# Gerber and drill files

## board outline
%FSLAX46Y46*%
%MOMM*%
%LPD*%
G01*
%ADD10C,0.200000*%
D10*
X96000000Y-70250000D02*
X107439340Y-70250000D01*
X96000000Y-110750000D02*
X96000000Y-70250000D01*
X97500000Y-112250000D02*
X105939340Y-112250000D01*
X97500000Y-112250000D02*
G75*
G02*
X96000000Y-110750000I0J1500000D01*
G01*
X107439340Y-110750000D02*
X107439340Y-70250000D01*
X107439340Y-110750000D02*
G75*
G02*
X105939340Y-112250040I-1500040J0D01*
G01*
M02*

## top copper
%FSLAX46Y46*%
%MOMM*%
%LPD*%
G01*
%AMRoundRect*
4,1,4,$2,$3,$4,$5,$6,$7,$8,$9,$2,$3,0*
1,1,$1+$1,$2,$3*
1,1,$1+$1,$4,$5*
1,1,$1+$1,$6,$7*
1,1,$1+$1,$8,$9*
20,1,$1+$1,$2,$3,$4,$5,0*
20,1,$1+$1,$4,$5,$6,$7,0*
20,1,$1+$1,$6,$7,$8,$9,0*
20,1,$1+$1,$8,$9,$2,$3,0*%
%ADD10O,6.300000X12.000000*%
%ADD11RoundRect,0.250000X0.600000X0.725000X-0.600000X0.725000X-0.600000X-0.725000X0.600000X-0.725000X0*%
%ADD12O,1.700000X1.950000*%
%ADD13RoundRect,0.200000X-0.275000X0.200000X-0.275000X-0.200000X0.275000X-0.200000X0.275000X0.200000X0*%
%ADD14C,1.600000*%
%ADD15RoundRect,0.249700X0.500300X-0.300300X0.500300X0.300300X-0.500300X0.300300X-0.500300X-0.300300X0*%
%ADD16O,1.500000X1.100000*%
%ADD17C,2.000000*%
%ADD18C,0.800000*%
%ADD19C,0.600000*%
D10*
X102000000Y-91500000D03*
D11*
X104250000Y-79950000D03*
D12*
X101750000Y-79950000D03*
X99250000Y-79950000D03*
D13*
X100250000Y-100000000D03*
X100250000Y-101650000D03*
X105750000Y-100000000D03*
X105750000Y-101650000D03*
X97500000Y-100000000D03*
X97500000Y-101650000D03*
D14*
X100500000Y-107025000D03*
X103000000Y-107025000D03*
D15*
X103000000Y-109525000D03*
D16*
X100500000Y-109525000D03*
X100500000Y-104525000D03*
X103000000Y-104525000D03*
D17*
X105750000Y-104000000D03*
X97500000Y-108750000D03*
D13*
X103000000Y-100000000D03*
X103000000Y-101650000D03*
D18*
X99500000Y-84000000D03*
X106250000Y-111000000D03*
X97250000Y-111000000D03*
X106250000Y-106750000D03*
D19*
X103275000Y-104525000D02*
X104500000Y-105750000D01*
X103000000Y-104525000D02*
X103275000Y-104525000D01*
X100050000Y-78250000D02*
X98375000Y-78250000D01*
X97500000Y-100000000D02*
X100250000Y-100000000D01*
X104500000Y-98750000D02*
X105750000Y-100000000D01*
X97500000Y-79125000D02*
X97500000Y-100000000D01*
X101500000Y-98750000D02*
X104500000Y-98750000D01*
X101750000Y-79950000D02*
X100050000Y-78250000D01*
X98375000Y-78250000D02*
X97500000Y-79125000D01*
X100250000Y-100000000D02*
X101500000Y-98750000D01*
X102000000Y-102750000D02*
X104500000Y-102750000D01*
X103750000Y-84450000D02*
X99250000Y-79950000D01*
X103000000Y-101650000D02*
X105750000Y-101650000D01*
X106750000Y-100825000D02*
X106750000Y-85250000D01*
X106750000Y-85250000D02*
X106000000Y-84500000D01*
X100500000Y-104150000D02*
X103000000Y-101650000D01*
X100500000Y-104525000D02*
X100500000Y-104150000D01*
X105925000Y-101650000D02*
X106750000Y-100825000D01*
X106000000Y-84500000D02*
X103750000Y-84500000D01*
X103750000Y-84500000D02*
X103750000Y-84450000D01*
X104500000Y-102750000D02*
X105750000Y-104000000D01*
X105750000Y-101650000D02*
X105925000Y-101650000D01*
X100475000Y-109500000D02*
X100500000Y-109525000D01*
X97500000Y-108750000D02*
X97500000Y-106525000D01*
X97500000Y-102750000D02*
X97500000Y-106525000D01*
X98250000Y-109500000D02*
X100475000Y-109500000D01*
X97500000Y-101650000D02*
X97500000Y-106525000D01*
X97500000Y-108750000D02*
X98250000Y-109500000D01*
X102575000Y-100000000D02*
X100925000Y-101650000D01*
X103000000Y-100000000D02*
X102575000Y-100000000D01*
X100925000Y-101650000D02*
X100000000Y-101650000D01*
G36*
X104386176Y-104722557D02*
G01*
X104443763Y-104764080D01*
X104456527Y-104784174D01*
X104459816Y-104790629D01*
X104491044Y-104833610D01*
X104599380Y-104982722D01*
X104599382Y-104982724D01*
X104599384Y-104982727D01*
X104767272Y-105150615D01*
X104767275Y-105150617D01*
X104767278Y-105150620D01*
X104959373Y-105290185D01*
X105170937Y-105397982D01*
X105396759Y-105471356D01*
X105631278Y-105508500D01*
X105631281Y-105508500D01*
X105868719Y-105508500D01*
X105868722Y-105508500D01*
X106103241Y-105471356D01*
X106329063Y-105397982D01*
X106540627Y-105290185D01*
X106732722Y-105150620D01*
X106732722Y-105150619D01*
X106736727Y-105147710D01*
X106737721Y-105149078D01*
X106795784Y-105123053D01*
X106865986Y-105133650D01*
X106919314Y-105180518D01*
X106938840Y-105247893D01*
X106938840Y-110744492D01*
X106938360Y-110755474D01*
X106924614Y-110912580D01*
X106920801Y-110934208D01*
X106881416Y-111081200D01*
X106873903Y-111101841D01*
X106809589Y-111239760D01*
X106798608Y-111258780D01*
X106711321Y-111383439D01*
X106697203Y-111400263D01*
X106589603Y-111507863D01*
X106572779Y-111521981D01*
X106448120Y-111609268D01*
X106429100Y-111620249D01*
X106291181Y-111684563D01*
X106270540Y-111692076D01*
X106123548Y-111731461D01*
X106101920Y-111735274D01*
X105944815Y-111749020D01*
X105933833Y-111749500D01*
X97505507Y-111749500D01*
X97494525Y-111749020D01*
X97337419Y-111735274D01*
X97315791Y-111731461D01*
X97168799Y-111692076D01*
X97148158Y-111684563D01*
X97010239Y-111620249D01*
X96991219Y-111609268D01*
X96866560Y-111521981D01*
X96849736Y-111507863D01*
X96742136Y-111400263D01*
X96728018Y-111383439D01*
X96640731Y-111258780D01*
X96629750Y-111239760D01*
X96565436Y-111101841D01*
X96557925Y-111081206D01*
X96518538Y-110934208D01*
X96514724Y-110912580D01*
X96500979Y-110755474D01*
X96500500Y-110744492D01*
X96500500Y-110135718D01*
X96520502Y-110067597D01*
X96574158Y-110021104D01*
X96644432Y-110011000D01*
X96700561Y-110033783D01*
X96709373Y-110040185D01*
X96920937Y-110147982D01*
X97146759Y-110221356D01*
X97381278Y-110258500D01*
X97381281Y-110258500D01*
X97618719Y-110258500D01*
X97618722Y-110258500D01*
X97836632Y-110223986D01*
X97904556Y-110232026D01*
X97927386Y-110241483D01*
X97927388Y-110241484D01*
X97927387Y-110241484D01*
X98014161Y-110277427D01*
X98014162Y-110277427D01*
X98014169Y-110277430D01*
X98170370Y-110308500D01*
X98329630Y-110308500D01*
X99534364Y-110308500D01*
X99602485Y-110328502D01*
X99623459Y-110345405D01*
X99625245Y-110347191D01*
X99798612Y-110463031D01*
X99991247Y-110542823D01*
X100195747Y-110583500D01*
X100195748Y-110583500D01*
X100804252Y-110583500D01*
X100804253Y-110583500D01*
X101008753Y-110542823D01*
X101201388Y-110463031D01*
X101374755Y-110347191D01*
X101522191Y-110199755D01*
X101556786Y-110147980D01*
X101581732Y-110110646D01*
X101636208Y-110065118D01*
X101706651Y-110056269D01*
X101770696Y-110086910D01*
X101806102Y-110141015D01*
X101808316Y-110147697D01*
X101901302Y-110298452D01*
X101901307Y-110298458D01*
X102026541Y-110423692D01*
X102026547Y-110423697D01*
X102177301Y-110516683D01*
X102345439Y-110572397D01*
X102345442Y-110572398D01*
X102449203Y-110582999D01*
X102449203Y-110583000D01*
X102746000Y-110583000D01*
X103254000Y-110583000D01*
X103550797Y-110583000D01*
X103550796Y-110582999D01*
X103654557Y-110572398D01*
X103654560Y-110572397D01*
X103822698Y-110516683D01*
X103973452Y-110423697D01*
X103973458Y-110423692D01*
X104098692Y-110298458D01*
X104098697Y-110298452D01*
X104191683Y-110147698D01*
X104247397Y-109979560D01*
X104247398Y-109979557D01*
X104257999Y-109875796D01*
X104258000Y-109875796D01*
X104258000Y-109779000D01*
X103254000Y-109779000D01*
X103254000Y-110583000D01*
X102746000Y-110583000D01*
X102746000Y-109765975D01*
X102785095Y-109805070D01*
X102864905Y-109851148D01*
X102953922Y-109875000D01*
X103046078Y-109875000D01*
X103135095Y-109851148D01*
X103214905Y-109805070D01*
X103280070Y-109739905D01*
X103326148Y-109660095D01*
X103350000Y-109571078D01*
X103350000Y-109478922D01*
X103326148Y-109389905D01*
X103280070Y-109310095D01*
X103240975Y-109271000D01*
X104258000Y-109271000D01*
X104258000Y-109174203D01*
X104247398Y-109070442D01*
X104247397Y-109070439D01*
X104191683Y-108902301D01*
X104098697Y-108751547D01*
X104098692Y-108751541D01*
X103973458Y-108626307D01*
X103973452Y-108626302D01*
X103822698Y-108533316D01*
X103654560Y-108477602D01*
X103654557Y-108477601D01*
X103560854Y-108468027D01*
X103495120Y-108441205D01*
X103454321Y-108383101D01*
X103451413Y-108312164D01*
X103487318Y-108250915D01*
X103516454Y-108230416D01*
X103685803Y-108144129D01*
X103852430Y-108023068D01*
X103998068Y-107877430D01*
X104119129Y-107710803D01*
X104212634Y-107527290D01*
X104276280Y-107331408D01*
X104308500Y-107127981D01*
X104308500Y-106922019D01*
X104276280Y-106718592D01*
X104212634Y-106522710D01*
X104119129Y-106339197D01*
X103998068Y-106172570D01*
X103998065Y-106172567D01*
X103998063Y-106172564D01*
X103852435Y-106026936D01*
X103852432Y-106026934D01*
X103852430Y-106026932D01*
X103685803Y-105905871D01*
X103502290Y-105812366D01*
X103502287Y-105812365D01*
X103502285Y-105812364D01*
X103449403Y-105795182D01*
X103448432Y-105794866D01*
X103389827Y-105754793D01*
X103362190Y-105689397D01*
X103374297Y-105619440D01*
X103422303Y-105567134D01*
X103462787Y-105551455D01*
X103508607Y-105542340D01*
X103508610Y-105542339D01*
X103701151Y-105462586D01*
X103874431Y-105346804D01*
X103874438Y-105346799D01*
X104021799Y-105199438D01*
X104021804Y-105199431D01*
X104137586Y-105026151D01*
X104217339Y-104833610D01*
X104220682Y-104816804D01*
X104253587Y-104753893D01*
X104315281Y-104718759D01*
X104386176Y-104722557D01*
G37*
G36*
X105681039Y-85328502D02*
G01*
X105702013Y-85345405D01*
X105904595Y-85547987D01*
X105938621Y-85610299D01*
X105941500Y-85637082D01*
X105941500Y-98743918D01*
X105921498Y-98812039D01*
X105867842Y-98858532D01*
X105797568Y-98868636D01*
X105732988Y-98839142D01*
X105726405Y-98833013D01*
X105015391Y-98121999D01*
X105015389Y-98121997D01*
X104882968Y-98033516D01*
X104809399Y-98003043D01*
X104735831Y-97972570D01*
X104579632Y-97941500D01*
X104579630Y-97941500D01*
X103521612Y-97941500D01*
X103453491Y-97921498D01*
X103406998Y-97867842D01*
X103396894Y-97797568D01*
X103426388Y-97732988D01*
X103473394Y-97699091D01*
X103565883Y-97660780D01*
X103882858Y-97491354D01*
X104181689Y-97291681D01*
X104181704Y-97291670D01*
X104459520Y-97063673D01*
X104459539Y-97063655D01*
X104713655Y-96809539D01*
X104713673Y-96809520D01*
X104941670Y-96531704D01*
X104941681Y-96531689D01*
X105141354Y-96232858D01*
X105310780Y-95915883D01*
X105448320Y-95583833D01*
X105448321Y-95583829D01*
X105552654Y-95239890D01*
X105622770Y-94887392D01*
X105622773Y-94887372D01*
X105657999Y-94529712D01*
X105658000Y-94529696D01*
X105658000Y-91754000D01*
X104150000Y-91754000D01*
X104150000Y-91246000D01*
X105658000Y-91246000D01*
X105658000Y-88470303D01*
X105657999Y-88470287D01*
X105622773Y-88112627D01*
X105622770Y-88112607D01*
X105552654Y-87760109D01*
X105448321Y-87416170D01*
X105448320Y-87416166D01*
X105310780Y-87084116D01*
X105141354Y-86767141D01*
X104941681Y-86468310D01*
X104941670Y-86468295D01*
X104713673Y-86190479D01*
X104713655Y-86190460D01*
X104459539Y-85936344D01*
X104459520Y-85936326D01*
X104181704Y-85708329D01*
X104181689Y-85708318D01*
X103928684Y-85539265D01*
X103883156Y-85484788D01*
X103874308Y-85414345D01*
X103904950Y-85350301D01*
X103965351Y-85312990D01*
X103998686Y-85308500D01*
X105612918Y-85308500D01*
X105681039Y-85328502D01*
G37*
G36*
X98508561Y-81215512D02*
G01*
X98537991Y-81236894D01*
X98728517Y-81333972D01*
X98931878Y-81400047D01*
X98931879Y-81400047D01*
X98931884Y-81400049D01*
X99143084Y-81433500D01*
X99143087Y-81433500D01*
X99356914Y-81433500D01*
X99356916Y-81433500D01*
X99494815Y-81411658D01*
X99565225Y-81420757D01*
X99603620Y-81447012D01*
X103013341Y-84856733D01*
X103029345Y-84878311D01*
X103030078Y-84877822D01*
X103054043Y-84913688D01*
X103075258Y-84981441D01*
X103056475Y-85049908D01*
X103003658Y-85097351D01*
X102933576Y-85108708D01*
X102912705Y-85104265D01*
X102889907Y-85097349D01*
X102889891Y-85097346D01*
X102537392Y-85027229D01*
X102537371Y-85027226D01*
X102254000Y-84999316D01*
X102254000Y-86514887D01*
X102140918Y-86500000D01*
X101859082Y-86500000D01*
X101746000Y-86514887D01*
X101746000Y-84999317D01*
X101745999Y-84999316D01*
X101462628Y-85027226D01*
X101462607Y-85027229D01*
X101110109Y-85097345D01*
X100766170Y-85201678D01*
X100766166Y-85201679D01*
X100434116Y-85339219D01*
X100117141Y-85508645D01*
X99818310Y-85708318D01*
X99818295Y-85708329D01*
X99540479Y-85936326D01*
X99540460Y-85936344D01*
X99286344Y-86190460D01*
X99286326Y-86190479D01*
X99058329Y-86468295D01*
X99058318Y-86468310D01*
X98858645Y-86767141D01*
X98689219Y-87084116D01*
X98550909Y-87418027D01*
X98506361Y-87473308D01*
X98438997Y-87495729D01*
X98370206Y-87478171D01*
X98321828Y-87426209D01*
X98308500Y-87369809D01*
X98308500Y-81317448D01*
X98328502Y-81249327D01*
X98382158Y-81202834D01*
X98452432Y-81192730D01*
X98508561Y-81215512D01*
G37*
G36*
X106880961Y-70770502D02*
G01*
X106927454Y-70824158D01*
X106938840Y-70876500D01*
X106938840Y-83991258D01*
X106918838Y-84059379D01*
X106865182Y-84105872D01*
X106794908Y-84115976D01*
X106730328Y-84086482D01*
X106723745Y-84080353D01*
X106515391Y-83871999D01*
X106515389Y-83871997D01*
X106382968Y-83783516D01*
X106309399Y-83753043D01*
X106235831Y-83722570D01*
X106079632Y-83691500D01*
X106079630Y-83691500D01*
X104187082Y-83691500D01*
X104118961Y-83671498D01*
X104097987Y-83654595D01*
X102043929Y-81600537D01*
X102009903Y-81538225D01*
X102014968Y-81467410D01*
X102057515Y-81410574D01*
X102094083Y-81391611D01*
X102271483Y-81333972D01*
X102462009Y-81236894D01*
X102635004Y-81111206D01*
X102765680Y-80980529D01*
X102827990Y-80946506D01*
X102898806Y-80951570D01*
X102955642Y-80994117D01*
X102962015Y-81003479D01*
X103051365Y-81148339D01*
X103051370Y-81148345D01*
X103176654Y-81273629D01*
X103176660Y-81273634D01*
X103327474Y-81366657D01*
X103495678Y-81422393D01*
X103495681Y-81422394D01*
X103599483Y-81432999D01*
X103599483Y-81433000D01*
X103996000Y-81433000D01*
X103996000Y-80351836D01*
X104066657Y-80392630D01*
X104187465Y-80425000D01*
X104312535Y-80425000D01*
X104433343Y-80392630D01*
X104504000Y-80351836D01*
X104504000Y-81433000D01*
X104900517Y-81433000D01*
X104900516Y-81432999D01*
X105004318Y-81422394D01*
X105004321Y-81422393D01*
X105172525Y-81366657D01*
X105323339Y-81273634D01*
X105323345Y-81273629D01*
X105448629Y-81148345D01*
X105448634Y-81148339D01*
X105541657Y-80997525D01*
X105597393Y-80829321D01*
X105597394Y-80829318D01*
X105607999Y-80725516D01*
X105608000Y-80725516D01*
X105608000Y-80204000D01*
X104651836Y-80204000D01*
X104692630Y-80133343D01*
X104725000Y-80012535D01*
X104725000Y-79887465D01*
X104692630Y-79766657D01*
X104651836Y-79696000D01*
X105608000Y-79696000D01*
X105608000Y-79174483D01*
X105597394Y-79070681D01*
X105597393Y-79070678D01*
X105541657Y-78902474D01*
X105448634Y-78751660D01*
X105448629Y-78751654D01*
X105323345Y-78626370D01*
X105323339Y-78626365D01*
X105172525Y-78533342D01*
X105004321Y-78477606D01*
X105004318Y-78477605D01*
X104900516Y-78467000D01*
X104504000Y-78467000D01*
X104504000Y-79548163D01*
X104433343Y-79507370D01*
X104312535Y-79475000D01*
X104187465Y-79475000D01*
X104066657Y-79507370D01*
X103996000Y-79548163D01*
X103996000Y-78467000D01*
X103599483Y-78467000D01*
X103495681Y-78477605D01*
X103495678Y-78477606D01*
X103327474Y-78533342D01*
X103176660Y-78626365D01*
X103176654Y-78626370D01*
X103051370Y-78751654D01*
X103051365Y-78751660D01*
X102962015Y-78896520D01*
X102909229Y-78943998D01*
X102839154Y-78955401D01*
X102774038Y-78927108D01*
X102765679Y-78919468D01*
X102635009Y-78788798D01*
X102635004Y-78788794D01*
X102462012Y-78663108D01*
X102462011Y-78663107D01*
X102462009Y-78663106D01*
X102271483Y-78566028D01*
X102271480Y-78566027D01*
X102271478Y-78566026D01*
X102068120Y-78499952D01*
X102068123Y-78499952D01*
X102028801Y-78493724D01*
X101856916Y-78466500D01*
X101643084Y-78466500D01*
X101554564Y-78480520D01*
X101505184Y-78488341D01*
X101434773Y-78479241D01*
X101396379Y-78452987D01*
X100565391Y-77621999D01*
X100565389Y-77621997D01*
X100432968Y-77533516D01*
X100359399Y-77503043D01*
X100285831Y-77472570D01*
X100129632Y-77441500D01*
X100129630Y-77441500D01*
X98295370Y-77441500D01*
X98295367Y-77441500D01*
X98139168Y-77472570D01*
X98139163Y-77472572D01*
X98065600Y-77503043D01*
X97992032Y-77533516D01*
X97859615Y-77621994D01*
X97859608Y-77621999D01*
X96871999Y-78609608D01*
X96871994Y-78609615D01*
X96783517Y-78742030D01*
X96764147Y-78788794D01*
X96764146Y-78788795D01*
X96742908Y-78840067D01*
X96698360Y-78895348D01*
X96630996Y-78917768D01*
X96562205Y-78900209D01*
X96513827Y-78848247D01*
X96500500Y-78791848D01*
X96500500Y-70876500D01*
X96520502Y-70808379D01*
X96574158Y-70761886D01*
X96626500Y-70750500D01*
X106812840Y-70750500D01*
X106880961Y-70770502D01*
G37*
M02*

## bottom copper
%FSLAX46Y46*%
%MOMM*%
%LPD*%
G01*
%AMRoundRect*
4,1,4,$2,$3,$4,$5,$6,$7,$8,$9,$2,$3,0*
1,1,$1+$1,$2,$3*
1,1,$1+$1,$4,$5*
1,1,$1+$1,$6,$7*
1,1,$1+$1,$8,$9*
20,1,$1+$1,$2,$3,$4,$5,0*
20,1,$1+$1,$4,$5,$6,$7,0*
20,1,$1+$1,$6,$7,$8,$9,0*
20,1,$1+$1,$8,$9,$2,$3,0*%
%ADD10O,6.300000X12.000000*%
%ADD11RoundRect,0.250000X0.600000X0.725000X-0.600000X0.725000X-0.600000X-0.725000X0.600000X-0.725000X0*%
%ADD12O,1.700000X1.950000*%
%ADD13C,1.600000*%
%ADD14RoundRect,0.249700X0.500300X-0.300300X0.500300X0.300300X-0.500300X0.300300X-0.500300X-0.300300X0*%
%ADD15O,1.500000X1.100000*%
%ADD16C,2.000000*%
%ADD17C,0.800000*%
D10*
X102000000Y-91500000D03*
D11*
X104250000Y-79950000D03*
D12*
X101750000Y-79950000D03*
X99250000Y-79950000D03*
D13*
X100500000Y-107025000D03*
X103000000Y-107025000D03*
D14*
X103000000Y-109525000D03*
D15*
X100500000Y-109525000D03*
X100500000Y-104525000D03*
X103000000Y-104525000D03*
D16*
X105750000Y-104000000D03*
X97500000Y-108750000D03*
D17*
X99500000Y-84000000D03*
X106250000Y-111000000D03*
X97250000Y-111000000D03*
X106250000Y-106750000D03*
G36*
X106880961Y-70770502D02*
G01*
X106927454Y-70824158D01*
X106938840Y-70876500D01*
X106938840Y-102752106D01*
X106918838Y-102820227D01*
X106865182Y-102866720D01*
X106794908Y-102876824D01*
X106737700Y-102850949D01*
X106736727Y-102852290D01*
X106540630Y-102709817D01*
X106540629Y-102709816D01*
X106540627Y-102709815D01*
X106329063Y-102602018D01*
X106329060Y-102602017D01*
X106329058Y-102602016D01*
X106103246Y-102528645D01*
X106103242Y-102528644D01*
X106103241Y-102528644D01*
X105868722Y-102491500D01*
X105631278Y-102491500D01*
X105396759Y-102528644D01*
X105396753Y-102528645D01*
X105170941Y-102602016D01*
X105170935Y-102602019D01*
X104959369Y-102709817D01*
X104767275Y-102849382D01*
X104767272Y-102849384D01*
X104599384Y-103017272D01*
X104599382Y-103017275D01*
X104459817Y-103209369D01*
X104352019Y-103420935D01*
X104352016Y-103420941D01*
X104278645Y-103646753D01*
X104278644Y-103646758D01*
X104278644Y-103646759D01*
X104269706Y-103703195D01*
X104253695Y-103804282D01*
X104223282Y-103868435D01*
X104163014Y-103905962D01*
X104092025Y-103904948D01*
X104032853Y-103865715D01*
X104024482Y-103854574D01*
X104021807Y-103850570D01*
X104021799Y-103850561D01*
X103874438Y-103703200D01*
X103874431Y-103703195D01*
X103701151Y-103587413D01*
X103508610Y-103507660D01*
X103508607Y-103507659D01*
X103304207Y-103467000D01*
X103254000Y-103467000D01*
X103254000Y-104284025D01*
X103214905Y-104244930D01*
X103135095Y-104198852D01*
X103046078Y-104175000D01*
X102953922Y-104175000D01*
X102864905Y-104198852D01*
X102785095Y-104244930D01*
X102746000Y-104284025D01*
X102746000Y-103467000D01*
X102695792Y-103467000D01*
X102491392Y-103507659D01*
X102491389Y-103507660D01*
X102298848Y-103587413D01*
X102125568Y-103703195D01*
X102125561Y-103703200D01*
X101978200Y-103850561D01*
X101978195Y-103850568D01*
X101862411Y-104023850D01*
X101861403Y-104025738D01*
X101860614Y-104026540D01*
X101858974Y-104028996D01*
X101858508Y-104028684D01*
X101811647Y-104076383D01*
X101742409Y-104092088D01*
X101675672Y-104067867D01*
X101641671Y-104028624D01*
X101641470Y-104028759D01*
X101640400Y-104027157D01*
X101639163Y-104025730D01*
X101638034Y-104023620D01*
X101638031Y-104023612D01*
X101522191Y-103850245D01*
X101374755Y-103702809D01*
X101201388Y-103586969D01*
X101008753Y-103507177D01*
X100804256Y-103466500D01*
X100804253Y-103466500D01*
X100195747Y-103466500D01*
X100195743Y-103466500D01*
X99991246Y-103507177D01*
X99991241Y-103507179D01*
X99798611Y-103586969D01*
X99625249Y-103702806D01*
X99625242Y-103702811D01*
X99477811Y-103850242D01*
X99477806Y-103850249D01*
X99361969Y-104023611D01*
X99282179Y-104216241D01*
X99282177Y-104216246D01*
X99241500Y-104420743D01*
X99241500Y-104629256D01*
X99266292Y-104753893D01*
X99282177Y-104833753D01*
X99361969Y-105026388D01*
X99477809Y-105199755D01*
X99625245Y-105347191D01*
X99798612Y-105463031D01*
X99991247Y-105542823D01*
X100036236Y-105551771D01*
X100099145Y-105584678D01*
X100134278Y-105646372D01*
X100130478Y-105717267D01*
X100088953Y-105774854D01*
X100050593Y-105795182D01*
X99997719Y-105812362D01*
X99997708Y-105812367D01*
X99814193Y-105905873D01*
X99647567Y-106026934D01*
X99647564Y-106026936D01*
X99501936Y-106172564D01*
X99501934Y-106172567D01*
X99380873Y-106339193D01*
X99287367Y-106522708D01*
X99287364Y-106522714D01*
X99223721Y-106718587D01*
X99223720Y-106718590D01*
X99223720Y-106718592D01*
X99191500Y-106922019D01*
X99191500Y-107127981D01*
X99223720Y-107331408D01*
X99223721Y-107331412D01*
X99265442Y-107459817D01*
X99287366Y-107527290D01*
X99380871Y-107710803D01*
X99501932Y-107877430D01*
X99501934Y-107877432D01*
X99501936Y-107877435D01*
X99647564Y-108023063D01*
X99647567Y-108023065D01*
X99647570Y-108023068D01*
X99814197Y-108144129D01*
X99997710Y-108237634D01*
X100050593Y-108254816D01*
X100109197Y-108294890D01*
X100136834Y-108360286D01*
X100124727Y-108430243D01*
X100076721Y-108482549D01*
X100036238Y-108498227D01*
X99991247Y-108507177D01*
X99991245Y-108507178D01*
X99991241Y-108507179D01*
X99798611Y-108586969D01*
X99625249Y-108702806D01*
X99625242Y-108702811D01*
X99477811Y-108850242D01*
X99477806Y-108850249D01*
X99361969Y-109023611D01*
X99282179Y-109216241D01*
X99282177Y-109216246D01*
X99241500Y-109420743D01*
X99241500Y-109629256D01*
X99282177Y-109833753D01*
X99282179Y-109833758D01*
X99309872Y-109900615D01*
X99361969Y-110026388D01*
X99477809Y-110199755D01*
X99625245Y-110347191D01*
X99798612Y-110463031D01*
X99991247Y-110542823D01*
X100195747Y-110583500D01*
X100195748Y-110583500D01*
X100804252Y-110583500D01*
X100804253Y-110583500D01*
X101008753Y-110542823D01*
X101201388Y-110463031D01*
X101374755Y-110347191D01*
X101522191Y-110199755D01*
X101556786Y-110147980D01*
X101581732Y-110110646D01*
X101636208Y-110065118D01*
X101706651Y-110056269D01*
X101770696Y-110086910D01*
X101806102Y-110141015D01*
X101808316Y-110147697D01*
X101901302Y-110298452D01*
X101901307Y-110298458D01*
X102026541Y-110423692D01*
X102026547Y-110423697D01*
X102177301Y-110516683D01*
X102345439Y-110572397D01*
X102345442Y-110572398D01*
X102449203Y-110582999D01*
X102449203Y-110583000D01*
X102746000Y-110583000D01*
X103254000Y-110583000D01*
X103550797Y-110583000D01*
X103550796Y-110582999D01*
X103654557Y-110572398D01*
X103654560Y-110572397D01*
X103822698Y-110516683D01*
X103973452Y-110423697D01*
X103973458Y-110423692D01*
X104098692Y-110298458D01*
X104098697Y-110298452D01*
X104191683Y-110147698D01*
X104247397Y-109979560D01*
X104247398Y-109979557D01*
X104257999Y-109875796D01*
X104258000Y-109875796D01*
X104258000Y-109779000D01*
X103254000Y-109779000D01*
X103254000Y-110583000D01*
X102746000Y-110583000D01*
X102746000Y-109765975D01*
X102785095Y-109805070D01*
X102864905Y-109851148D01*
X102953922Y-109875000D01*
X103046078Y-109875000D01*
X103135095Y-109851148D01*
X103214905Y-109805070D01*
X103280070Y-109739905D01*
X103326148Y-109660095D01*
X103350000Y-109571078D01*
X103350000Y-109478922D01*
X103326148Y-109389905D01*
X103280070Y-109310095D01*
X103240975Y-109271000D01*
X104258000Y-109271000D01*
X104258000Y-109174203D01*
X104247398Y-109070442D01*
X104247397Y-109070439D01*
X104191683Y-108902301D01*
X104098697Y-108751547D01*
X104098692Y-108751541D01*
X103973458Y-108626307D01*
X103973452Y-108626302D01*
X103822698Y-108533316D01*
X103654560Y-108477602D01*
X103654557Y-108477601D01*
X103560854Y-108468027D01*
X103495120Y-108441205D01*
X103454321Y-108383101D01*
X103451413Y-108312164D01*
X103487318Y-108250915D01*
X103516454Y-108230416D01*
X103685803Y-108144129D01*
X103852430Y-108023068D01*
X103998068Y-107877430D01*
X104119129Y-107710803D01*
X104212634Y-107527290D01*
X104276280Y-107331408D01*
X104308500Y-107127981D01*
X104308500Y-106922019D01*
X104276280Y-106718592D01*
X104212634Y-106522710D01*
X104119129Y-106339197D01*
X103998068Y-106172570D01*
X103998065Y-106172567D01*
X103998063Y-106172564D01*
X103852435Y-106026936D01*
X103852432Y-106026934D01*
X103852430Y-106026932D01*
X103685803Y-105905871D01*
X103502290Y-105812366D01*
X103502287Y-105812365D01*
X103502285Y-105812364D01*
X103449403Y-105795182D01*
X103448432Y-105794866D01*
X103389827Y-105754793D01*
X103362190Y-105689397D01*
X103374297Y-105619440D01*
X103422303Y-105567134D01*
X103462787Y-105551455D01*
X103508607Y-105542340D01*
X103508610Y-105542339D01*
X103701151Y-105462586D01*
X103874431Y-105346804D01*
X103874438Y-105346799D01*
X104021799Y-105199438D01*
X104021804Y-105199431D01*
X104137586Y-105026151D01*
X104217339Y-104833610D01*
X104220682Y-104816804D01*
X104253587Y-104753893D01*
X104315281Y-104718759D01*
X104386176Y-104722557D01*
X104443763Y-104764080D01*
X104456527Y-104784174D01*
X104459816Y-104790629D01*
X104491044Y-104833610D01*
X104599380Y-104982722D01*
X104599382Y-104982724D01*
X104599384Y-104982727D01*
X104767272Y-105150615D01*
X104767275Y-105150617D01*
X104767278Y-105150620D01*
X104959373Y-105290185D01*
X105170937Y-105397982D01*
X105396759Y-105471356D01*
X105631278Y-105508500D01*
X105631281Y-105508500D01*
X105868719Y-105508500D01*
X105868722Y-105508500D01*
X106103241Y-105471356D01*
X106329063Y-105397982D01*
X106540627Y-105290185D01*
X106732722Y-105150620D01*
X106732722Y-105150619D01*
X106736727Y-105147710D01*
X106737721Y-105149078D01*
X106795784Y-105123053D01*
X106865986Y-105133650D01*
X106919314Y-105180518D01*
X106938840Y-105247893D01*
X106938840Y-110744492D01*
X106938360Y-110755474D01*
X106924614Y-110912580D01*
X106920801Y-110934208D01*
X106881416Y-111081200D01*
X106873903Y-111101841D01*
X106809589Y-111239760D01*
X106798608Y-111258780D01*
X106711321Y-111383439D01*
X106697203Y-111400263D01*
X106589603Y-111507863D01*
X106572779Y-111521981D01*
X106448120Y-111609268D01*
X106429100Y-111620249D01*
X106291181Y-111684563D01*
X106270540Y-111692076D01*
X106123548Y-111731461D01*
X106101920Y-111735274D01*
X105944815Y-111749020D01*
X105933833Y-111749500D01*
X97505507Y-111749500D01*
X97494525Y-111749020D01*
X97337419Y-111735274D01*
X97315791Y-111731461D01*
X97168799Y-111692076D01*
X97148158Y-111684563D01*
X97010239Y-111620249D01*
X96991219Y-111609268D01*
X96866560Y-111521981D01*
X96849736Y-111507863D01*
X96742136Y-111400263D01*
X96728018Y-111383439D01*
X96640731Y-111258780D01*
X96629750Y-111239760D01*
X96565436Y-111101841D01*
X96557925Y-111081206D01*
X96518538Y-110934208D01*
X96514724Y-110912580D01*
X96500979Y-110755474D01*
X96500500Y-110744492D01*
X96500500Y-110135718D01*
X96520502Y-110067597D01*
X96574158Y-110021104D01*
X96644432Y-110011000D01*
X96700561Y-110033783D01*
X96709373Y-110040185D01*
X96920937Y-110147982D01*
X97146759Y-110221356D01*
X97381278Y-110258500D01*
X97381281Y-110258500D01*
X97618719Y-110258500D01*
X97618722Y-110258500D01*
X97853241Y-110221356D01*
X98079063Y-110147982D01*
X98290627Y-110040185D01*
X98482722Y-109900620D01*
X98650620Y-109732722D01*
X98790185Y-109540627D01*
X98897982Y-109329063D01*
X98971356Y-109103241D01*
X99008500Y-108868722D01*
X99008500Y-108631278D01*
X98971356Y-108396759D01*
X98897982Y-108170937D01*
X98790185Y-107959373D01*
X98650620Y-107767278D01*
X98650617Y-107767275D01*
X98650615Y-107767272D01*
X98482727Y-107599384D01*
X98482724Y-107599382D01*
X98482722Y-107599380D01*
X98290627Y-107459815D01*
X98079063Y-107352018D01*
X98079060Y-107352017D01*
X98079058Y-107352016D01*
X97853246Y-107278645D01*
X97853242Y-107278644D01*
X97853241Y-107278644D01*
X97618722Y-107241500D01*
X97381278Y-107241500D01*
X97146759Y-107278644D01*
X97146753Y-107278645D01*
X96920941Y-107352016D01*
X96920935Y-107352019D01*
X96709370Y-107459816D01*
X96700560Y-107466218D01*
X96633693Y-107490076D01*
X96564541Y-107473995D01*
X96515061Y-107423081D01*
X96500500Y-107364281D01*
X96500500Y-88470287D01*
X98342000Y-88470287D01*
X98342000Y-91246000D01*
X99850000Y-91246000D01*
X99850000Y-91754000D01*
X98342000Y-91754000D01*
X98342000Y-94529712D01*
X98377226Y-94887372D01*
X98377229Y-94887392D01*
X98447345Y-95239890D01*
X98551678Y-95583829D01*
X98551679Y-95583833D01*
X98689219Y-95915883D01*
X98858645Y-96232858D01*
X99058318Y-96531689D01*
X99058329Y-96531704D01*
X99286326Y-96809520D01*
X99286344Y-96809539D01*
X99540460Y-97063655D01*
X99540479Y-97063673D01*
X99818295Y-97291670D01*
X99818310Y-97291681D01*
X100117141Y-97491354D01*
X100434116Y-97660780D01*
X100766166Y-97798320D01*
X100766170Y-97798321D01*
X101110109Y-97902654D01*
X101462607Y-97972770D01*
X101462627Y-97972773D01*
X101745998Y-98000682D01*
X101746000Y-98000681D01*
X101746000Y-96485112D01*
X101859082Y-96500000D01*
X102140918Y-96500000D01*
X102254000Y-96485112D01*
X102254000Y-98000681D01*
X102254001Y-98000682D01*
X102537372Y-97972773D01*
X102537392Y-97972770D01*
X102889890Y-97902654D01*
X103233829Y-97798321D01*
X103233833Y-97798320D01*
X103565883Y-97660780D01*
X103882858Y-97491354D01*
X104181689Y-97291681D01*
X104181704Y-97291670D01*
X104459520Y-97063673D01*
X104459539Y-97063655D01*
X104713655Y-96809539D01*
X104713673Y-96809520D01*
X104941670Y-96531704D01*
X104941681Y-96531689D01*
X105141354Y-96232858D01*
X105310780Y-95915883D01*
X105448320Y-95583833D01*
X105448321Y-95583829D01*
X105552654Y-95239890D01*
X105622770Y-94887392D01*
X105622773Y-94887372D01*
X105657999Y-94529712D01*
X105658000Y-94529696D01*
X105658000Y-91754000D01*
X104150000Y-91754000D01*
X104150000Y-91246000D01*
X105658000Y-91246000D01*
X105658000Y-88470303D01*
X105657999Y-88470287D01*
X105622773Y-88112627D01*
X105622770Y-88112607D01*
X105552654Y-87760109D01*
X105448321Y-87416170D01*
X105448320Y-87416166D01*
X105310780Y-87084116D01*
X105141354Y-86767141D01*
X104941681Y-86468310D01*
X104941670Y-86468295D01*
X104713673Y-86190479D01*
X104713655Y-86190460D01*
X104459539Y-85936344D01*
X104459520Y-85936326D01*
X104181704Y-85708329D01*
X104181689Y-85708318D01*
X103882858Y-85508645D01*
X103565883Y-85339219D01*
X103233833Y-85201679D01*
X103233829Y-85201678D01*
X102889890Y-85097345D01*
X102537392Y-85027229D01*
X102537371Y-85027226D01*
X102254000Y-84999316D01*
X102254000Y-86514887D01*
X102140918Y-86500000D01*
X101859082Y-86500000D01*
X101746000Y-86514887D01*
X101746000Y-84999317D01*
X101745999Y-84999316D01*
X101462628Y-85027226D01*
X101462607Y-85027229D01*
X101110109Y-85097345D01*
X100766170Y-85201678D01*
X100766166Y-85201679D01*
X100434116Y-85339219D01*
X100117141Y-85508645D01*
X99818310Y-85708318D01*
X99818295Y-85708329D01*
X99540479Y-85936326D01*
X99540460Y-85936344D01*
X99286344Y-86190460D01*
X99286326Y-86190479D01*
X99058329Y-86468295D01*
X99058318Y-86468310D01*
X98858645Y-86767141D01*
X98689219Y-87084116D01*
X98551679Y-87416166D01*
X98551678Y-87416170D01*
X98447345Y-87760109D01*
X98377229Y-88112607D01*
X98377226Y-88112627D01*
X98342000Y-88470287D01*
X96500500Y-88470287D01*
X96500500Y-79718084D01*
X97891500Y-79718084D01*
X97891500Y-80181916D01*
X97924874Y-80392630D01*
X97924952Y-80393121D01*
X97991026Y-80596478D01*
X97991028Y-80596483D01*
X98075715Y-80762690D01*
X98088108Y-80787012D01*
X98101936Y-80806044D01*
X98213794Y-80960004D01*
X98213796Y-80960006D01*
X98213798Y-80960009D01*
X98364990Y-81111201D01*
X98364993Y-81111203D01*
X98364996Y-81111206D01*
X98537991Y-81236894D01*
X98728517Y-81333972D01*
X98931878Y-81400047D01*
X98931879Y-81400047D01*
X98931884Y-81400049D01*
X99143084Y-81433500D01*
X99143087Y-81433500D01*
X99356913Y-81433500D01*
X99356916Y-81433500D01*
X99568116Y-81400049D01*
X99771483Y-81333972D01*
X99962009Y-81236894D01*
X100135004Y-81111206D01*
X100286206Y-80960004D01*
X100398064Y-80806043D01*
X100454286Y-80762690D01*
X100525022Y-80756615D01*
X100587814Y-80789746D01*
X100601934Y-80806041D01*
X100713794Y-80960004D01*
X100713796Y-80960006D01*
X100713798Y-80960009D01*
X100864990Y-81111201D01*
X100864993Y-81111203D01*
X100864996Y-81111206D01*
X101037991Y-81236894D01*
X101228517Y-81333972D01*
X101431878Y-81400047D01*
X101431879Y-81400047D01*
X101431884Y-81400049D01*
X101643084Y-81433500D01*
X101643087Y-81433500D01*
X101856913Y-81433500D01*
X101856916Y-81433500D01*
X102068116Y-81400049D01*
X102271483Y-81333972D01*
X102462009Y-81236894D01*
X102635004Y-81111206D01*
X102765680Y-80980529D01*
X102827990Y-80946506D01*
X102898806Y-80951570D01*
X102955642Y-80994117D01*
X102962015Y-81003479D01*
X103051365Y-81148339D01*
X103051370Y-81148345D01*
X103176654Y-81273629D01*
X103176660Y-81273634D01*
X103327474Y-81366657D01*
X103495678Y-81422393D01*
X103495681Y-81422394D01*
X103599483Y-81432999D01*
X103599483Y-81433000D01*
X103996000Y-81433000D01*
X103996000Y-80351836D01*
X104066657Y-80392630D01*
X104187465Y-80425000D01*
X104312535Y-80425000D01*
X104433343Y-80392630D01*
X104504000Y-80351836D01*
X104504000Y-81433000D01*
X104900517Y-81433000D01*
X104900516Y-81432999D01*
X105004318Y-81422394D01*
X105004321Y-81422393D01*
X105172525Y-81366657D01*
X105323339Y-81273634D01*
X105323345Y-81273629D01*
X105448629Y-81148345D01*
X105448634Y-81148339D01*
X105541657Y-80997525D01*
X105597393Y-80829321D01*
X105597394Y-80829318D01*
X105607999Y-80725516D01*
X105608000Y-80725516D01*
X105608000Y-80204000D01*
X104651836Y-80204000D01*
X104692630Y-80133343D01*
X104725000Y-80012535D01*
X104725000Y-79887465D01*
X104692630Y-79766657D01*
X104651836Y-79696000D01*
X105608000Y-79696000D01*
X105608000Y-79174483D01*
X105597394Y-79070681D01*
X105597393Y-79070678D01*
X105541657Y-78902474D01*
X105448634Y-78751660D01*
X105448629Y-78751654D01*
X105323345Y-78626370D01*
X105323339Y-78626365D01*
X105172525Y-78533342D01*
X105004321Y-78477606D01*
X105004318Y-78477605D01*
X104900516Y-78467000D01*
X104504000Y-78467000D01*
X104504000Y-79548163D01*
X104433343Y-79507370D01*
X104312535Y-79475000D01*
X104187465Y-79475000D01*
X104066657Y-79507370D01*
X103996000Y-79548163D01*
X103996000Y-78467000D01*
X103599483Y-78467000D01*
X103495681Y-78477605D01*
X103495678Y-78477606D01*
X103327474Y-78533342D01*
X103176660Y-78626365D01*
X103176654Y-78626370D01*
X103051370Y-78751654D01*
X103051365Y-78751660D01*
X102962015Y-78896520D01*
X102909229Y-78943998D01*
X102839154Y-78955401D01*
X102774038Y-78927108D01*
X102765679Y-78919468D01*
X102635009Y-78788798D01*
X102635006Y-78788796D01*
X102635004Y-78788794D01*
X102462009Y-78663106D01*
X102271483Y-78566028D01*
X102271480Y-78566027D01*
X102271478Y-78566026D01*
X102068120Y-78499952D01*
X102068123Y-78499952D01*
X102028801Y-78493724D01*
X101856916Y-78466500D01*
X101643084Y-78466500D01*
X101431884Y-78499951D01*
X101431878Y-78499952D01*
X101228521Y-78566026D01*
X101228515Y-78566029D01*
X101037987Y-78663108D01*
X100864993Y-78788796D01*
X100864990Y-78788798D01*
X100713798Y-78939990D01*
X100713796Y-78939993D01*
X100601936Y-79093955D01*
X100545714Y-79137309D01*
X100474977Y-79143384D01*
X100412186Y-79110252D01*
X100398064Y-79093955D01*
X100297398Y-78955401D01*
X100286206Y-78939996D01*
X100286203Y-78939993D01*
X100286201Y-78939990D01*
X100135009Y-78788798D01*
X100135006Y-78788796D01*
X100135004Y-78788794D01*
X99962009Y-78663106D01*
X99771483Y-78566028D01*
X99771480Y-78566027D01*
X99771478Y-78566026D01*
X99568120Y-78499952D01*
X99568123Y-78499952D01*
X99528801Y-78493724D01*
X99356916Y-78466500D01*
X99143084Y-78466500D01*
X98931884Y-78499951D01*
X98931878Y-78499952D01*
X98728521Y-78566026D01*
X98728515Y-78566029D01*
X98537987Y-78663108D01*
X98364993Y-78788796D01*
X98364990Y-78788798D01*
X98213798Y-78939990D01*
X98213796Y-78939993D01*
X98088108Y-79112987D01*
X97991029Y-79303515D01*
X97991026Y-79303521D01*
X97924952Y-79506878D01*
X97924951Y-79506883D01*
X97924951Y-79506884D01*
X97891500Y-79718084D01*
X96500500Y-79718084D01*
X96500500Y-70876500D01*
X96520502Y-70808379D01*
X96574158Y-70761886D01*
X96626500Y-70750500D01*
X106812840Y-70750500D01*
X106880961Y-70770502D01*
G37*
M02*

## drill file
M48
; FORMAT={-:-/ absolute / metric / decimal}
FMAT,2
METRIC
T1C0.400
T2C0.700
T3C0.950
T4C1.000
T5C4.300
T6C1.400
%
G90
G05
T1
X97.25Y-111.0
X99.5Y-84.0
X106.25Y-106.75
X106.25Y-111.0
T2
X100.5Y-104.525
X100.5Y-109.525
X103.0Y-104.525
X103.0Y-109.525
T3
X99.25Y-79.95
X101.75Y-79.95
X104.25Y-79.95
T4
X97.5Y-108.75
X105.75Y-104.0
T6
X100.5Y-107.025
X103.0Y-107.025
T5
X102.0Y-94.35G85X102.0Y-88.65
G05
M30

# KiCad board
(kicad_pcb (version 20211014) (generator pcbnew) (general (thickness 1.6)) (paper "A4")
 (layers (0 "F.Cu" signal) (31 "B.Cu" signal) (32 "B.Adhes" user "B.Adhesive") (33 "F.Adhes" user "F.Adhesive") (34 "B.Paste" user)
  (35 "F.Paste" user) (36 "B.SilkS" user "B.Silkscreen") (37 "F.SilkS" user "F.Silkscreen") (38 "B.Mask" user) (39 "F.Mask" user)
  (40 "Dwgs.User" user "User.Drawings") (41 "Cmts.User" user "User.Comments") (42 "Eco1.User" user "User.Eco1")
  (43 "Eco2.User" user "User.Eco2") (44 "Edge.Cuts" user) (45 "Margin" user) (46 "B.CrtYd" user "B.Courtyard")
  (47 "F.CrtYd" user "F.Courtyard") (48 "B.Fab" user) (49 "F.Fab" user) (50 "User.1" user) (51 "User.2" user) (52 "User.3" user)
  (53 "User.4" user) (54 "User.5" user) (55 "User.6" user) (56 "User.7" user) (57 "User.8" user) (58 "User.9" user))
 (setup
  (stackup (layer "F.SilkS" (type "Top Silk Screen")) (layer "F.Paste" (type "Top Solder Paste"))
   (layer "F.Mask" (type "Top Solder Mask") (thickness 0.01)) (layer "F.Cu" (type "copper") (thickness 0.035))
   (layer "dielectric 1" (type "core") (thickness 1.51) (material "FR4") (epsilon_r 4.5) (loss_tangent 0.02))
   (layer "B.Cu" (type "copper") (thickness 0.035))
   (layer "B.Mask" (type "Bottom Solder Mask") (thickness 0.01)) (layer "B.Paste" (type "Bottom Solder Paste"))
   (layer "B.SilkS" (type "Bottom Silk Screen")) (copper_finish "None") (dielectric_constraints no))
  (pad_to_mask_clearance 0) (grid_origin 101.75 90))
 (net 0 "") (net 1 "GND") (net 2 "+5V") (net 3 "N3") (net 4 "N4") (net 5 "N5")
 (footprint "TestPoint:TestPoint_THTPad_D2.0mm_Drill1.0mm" (layer "F.Cu") (at 102 91.5 180)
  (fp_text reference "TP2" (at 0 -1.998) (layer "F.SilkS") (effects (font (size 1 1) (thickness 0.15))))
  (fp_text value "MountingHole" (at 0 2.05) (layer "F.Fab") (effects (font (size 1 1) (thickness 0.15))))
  (pad "1" thru_hole oval (at 0 0 180) (size 6.3 12) (drill oval 4.3 10) (layers *.Cu *.Mask) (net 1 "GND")))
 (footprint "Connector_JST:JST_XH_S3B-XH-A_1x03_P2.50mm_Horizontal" (layer "F.Cu") (at 104.25 79.95 180)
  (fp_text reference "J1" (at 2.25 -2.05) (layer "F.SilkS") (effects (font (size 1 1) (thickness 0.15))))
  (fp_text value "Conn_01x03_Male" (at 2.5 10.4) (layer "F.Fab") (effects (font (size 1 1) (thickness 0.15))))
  (pad "1" thru_hole roundrect (at 0 0 180) (size 1.7 1.95) (drill 0.95) (layers *.Cu *.Mask) (roundrect_rratio 0.1470588235) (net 1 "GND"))
  (pad "2" thru_hole oval (at 2.5 0 180) (size 1.7 1.95) (drill 0.95) (layers *.Cu *.Mask) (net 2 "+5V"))
  (pad "3" thru_hole oval (at 5 0 180) (size 1.7 1.95) (drill 0.95) (layers *.Cu *.Mask) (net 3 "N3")))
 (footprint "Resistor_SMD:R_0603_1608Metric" (layer "F.Cu") (at 100.25 100.825 -90)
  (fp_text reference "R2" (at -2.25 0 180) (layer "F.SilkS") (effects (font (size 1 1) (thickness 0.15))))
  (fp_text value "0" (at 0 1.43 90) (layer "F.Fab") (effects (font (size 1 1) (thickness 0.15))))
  (pad "1" smd roundrect (at -0.825 0 270) (size 0.8 0.95) (layers "F.Cu" "F.Paste" "F.Mask") (roundrect_rratio 0.25) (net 2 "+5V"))
  (pad "2" smd roundrect (at 0.825 0 270) (size 0.8 0.95) (layers "F.Cu" "F.Paste" "F.Mask") (roundrect_rratio 0.25) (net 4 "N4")))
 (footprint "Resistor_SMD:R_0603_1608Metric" (layer "F.Cu") (at 105.75 100.825 -90)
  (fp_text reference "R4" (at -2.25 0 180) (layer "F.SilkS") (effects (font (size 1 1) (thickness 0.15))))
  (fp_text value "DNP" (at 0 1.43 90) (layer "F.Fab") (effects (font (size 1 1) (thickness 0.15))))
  (pad "1" smd roundrect (at -0.825 0 270) (size 0.8 0.95) (layers "F.Cu" "F.Paste" "F.Mask") (roundrect_rratio 0.25) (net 2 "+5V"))
  (pad "2" smd roundrect (at 0.825 0 270) (size 0.8 0.95) (layers "F.Cu" "F.Paste" "F.Mask") (roundrect_rratio 0.25) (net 3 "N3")))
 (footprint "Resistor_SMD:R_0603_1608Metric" (layer "F.Cu") (at 97.5 100.825 -90)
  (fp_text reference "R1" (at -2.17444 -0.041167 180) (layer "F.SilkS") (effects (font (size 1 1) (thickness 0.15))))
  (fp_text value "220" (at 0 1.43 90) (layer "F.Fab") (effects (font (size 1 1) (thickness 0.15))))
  (pad "1" smd roundrect (at -0.825 0 270) (size 0.8 0.95) (layers "F.Cu" "F.Paste" "F.Mask") (roundrect_rratio 0.25) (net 2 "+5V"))
  (pad "2" smd roundrect (at 0.825 0 270) (size 0.8 0.95) (layers "F.Cu" "F.Paste" "F.Mask") (roundrect_rratio 0.25) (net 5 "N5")))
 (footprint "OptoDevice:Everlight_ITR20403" (layer "F.Cu") (at 103 109.525 90)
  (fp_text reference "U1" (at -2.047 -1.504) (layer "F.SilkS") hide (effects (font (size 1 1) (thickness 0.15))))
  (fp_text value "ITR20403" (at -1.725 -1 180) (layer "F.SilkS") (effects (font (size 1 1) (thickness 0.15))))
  (pad "" np_thru_hole circle (at 2.5 -2.5 90) (size 1.6 1.6) (drill 1.4) (layers F&B.Cu *.Mask))
  (pad "" np_thru_hole circle (at 2.5 0 90) (size 1.6 1.6) (drill 1.4) (layers F&B.Cu *.Mask))
  (pad "1" thru_hole roundrect (at 0 0 90) (size 1.1 1.5) (drill 0.7) (layers *.Cu *.Mask) (roundrect_rratio 0.227) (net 1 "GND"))
  (pad "2" thru_hole oval (at 0 -2.5 90) (size 1.1 1.5) (drill 0.7) (layers *.Cu *.Mask) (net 5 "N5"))
  (pad "3" thru_hole oval (at 5 -2.5 90) (size 1.1 1.5) (drill 0.7) (layers *.Cu *.Mask) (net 3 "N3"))
  (pad "4" thru_hole oval (at 5 0 90) (size 1.1 1.5) (drill 0.7) (layers *.Cu *.Mask) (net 1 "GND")))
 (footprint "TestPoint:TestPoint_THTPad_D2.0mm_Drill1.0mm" (layer "F.Cu") (at 105.75 104)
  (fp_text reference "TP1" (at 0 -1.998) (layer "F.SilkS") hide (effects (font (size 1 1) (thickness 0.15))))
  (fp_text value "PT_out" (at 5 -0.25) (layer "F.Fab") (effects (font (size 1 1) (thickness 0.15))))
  (pad "1" thru_hole circle (at 0 0) (size 2 2) (drill 1) (layers *.Cu *.Mask) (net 3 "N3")))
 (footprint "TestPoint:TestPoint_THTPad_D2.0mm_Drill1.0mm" (layer "F.Cu") (at 97.5 108.75)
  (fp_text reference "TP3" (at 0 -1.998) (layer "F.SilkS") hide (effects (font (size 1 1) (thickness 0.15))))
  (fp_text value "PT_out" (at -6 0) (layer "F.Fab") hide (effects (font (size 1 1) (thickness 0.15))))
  (pad "1" thru_hole circle (at 0 0) (size 2 2) (drill 1) (layers *.Cu *.Mask) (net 5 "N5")))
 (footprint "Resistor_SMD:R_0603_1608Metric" (layer "F.Cu") (at 103 100.825 -90)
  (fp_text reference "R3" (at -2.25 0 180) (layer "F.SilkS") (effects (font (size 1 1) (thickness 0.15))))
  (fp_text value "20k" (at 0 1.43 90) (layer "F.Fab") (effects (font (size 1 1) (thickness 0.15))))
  (pad "1" smd roundrect (at -0.825 0 270) (size 0.8 0.95) (layers "F.Cu" "F.Paste" "F.Mask") (roundrect_rratio 0.25) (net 4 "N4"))
  (pad "2" smd roundrect (at 0.825 0 270) (size 0.8 0.95) (layers "F.Cu" "F.Paste" "F.Mask") (roundrect_rratio 0.25) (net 3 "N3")))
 (gr_line (start 96 70.25) (end 107.43934 70.25) (layer "Edge.Cuts") (width 0.2))
 (gr_line (start 96 110.75) (end 96 70.25) (layer "Edge.Cuts") (width 0.2))
 (gr_line (start 97.5 112.25) (end 105.93934 112.25) (layer "Edge.Cuts") (width 0.2))
 (gr_arc (start 97.5 112.25) (mid 96.43934 111.81066) (end 96 110.75) (layer "Edge.Cuts") (width 0.2))
 (gr_line (start 107.43934 110.75) (end 107.43934 70.25) (layer "Edge.Cuts") (width 0.2))
 (gr_arc (start 107.43934 110.75) (mid 107 111.81066) (end 105.93934 112.25) (layer "Edge.Cuts") (width 0.2))
 (segment (start 103.275 104.525) (end 104.5 105.75) (width 0.6) (layer "F.Cu") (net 1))
 (segment (start 103 104.525) (end 103.275 104.525) (width 0.6) (layer "F.Cu") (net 1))
 (via (at 99.5 84) (size 0.8) (drill 0.4) (layers "F.Cu" "B.Cu") (free) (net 1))
 (via (at 106.25 111) (size 0.8) (drill 0.4) (layers "F.Cu" "B.Cu") (free) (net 1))
 (via (at 97.25 111) (size 0.8) (drill 0.4) (layers "F.Cu" "B.Cu") (free) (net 1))
 (via (at 106.25 106.75) (size 0.8) (drill 0.4) (layers "F.Cu" "B.Cu") (free) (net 1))
 (segment (start 100.05 78.25) (end 98.375 78.25) (width 0.6) (layer "F.Cu") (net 2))
 (segment (start 97.5 100) (end 100.25 100) (width 0.6) (layer "F.Cu") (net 2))
 (segment (start 104.5 98.75) (end 105.75 100) (width 0.6) (layer "F.Cu") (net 2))
 (segment (start 97.5 79.125) (end 97.5 100) (width 0.6) (layer "F.Cu") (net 2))
 (segment (start 101.5 98.75) (end 104.5 98.75) (width 0.6) (layer "F.Cu") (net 2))
 (segment (start 101.75 79.95) (end 100.05 78.25) (width 0.6) (layer "F.Cu") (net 2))
 (segment (start 98.375 78.25) (end 97.5 79.125) (width 0.6) (layer "F.Cu") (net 2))
 (segment (start 100.25 100) (end 101.5 98.75) (width 0.6) (layer "F.Cu") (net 2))
 (segment (start 102 102.75) (end 104.5 102.75) (width 0.6) (layer "F.Cu") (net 3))
 (segment (start 103.75 84.45) (end 99.25 79.95) (width 0.6) (layer "F.Cu") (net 3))
 (segment (start 103 101.65) (end 105.75 101.65) (width 0.6) (layer "F.Cu") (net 3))
 (segment (start 106.75 100.825) (end 106.75 85.25) (width 0.6) (layer "F.Cu") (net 3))
 (segment (start 106.75 85.25) (end 106 84.5) (width 0.6) (layer "F.Cu") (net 3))
 (segment (start 100.5 104.15) (end 103 101.65) (width 0.6) (layer "F.Cu") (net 3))
 (segment (start 100.5 104.525) (end 100.5 104.15) (width 0.6) (layer "F.Cu") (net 3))
 (segment (start 105.925 101.65) (end 106.75 100.825) (width 0.6) (layer "F.Cu") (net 3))
 (segment (start 106 84.5) (end 103.75 84.5) (width 0.6) (layer "F.Cu") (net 3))
 (segment (start 103.75 84.5) (end 103.75 84.45) (width 0.6) (layer "F.Cu") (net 3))
 (segment (start 104.5 102.75) (end 105.75 104) (width 0.6) (layer "F.Cu") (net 3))
 (segment (start 105.75 101.65) (end 105.925 101.65) (width 0.6) (layer "F.Cu") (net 3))
 (segment (start 100.475 109.5) (end 100.5 109.525) (width 0.6) (layer "F.Cu") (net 5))
 (segment (start 97.5 108.75) (end 97.5 106.525) (width 0.6) (layer "F.Cu") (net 5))
 (segment (start 97.5 102.75) (end 97.5 106.525) (width 0.6) (layer "F.Cu") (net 5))
 (segment (start 98.25 109.5) (end 100.475 109.5) (width 0.6) (layer "F.Cu") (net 5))
 (segment (start 97.5 101.65) (end 97.5 106.525) (width 0.6) (layer "F.Cu") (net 5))
 (segment (start 97.5 108.75) (end 98.25 109.5) (width 0.6) (layer "F.Cu") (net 5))
 (segment (start 102.575 100) (end 100.925 101.65) (width 0.6) (layer "F.Cu") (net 4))
 (segment (start 103 100) (end 102.575 100) (width 0.6) (layer "F.Cu") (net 4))
 (segment (start 100.925 101.65) (end 100 101.65) (width 0.6) (layer "F.Cu") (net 4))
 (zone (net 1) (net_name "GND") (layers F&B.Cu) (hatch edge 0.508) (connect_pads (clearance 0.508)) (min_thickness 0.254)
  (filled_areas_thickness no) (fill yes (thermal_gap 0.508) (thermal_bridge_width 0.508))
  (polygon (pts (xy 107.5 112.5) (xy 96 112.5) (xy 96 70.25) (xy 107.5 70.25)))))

